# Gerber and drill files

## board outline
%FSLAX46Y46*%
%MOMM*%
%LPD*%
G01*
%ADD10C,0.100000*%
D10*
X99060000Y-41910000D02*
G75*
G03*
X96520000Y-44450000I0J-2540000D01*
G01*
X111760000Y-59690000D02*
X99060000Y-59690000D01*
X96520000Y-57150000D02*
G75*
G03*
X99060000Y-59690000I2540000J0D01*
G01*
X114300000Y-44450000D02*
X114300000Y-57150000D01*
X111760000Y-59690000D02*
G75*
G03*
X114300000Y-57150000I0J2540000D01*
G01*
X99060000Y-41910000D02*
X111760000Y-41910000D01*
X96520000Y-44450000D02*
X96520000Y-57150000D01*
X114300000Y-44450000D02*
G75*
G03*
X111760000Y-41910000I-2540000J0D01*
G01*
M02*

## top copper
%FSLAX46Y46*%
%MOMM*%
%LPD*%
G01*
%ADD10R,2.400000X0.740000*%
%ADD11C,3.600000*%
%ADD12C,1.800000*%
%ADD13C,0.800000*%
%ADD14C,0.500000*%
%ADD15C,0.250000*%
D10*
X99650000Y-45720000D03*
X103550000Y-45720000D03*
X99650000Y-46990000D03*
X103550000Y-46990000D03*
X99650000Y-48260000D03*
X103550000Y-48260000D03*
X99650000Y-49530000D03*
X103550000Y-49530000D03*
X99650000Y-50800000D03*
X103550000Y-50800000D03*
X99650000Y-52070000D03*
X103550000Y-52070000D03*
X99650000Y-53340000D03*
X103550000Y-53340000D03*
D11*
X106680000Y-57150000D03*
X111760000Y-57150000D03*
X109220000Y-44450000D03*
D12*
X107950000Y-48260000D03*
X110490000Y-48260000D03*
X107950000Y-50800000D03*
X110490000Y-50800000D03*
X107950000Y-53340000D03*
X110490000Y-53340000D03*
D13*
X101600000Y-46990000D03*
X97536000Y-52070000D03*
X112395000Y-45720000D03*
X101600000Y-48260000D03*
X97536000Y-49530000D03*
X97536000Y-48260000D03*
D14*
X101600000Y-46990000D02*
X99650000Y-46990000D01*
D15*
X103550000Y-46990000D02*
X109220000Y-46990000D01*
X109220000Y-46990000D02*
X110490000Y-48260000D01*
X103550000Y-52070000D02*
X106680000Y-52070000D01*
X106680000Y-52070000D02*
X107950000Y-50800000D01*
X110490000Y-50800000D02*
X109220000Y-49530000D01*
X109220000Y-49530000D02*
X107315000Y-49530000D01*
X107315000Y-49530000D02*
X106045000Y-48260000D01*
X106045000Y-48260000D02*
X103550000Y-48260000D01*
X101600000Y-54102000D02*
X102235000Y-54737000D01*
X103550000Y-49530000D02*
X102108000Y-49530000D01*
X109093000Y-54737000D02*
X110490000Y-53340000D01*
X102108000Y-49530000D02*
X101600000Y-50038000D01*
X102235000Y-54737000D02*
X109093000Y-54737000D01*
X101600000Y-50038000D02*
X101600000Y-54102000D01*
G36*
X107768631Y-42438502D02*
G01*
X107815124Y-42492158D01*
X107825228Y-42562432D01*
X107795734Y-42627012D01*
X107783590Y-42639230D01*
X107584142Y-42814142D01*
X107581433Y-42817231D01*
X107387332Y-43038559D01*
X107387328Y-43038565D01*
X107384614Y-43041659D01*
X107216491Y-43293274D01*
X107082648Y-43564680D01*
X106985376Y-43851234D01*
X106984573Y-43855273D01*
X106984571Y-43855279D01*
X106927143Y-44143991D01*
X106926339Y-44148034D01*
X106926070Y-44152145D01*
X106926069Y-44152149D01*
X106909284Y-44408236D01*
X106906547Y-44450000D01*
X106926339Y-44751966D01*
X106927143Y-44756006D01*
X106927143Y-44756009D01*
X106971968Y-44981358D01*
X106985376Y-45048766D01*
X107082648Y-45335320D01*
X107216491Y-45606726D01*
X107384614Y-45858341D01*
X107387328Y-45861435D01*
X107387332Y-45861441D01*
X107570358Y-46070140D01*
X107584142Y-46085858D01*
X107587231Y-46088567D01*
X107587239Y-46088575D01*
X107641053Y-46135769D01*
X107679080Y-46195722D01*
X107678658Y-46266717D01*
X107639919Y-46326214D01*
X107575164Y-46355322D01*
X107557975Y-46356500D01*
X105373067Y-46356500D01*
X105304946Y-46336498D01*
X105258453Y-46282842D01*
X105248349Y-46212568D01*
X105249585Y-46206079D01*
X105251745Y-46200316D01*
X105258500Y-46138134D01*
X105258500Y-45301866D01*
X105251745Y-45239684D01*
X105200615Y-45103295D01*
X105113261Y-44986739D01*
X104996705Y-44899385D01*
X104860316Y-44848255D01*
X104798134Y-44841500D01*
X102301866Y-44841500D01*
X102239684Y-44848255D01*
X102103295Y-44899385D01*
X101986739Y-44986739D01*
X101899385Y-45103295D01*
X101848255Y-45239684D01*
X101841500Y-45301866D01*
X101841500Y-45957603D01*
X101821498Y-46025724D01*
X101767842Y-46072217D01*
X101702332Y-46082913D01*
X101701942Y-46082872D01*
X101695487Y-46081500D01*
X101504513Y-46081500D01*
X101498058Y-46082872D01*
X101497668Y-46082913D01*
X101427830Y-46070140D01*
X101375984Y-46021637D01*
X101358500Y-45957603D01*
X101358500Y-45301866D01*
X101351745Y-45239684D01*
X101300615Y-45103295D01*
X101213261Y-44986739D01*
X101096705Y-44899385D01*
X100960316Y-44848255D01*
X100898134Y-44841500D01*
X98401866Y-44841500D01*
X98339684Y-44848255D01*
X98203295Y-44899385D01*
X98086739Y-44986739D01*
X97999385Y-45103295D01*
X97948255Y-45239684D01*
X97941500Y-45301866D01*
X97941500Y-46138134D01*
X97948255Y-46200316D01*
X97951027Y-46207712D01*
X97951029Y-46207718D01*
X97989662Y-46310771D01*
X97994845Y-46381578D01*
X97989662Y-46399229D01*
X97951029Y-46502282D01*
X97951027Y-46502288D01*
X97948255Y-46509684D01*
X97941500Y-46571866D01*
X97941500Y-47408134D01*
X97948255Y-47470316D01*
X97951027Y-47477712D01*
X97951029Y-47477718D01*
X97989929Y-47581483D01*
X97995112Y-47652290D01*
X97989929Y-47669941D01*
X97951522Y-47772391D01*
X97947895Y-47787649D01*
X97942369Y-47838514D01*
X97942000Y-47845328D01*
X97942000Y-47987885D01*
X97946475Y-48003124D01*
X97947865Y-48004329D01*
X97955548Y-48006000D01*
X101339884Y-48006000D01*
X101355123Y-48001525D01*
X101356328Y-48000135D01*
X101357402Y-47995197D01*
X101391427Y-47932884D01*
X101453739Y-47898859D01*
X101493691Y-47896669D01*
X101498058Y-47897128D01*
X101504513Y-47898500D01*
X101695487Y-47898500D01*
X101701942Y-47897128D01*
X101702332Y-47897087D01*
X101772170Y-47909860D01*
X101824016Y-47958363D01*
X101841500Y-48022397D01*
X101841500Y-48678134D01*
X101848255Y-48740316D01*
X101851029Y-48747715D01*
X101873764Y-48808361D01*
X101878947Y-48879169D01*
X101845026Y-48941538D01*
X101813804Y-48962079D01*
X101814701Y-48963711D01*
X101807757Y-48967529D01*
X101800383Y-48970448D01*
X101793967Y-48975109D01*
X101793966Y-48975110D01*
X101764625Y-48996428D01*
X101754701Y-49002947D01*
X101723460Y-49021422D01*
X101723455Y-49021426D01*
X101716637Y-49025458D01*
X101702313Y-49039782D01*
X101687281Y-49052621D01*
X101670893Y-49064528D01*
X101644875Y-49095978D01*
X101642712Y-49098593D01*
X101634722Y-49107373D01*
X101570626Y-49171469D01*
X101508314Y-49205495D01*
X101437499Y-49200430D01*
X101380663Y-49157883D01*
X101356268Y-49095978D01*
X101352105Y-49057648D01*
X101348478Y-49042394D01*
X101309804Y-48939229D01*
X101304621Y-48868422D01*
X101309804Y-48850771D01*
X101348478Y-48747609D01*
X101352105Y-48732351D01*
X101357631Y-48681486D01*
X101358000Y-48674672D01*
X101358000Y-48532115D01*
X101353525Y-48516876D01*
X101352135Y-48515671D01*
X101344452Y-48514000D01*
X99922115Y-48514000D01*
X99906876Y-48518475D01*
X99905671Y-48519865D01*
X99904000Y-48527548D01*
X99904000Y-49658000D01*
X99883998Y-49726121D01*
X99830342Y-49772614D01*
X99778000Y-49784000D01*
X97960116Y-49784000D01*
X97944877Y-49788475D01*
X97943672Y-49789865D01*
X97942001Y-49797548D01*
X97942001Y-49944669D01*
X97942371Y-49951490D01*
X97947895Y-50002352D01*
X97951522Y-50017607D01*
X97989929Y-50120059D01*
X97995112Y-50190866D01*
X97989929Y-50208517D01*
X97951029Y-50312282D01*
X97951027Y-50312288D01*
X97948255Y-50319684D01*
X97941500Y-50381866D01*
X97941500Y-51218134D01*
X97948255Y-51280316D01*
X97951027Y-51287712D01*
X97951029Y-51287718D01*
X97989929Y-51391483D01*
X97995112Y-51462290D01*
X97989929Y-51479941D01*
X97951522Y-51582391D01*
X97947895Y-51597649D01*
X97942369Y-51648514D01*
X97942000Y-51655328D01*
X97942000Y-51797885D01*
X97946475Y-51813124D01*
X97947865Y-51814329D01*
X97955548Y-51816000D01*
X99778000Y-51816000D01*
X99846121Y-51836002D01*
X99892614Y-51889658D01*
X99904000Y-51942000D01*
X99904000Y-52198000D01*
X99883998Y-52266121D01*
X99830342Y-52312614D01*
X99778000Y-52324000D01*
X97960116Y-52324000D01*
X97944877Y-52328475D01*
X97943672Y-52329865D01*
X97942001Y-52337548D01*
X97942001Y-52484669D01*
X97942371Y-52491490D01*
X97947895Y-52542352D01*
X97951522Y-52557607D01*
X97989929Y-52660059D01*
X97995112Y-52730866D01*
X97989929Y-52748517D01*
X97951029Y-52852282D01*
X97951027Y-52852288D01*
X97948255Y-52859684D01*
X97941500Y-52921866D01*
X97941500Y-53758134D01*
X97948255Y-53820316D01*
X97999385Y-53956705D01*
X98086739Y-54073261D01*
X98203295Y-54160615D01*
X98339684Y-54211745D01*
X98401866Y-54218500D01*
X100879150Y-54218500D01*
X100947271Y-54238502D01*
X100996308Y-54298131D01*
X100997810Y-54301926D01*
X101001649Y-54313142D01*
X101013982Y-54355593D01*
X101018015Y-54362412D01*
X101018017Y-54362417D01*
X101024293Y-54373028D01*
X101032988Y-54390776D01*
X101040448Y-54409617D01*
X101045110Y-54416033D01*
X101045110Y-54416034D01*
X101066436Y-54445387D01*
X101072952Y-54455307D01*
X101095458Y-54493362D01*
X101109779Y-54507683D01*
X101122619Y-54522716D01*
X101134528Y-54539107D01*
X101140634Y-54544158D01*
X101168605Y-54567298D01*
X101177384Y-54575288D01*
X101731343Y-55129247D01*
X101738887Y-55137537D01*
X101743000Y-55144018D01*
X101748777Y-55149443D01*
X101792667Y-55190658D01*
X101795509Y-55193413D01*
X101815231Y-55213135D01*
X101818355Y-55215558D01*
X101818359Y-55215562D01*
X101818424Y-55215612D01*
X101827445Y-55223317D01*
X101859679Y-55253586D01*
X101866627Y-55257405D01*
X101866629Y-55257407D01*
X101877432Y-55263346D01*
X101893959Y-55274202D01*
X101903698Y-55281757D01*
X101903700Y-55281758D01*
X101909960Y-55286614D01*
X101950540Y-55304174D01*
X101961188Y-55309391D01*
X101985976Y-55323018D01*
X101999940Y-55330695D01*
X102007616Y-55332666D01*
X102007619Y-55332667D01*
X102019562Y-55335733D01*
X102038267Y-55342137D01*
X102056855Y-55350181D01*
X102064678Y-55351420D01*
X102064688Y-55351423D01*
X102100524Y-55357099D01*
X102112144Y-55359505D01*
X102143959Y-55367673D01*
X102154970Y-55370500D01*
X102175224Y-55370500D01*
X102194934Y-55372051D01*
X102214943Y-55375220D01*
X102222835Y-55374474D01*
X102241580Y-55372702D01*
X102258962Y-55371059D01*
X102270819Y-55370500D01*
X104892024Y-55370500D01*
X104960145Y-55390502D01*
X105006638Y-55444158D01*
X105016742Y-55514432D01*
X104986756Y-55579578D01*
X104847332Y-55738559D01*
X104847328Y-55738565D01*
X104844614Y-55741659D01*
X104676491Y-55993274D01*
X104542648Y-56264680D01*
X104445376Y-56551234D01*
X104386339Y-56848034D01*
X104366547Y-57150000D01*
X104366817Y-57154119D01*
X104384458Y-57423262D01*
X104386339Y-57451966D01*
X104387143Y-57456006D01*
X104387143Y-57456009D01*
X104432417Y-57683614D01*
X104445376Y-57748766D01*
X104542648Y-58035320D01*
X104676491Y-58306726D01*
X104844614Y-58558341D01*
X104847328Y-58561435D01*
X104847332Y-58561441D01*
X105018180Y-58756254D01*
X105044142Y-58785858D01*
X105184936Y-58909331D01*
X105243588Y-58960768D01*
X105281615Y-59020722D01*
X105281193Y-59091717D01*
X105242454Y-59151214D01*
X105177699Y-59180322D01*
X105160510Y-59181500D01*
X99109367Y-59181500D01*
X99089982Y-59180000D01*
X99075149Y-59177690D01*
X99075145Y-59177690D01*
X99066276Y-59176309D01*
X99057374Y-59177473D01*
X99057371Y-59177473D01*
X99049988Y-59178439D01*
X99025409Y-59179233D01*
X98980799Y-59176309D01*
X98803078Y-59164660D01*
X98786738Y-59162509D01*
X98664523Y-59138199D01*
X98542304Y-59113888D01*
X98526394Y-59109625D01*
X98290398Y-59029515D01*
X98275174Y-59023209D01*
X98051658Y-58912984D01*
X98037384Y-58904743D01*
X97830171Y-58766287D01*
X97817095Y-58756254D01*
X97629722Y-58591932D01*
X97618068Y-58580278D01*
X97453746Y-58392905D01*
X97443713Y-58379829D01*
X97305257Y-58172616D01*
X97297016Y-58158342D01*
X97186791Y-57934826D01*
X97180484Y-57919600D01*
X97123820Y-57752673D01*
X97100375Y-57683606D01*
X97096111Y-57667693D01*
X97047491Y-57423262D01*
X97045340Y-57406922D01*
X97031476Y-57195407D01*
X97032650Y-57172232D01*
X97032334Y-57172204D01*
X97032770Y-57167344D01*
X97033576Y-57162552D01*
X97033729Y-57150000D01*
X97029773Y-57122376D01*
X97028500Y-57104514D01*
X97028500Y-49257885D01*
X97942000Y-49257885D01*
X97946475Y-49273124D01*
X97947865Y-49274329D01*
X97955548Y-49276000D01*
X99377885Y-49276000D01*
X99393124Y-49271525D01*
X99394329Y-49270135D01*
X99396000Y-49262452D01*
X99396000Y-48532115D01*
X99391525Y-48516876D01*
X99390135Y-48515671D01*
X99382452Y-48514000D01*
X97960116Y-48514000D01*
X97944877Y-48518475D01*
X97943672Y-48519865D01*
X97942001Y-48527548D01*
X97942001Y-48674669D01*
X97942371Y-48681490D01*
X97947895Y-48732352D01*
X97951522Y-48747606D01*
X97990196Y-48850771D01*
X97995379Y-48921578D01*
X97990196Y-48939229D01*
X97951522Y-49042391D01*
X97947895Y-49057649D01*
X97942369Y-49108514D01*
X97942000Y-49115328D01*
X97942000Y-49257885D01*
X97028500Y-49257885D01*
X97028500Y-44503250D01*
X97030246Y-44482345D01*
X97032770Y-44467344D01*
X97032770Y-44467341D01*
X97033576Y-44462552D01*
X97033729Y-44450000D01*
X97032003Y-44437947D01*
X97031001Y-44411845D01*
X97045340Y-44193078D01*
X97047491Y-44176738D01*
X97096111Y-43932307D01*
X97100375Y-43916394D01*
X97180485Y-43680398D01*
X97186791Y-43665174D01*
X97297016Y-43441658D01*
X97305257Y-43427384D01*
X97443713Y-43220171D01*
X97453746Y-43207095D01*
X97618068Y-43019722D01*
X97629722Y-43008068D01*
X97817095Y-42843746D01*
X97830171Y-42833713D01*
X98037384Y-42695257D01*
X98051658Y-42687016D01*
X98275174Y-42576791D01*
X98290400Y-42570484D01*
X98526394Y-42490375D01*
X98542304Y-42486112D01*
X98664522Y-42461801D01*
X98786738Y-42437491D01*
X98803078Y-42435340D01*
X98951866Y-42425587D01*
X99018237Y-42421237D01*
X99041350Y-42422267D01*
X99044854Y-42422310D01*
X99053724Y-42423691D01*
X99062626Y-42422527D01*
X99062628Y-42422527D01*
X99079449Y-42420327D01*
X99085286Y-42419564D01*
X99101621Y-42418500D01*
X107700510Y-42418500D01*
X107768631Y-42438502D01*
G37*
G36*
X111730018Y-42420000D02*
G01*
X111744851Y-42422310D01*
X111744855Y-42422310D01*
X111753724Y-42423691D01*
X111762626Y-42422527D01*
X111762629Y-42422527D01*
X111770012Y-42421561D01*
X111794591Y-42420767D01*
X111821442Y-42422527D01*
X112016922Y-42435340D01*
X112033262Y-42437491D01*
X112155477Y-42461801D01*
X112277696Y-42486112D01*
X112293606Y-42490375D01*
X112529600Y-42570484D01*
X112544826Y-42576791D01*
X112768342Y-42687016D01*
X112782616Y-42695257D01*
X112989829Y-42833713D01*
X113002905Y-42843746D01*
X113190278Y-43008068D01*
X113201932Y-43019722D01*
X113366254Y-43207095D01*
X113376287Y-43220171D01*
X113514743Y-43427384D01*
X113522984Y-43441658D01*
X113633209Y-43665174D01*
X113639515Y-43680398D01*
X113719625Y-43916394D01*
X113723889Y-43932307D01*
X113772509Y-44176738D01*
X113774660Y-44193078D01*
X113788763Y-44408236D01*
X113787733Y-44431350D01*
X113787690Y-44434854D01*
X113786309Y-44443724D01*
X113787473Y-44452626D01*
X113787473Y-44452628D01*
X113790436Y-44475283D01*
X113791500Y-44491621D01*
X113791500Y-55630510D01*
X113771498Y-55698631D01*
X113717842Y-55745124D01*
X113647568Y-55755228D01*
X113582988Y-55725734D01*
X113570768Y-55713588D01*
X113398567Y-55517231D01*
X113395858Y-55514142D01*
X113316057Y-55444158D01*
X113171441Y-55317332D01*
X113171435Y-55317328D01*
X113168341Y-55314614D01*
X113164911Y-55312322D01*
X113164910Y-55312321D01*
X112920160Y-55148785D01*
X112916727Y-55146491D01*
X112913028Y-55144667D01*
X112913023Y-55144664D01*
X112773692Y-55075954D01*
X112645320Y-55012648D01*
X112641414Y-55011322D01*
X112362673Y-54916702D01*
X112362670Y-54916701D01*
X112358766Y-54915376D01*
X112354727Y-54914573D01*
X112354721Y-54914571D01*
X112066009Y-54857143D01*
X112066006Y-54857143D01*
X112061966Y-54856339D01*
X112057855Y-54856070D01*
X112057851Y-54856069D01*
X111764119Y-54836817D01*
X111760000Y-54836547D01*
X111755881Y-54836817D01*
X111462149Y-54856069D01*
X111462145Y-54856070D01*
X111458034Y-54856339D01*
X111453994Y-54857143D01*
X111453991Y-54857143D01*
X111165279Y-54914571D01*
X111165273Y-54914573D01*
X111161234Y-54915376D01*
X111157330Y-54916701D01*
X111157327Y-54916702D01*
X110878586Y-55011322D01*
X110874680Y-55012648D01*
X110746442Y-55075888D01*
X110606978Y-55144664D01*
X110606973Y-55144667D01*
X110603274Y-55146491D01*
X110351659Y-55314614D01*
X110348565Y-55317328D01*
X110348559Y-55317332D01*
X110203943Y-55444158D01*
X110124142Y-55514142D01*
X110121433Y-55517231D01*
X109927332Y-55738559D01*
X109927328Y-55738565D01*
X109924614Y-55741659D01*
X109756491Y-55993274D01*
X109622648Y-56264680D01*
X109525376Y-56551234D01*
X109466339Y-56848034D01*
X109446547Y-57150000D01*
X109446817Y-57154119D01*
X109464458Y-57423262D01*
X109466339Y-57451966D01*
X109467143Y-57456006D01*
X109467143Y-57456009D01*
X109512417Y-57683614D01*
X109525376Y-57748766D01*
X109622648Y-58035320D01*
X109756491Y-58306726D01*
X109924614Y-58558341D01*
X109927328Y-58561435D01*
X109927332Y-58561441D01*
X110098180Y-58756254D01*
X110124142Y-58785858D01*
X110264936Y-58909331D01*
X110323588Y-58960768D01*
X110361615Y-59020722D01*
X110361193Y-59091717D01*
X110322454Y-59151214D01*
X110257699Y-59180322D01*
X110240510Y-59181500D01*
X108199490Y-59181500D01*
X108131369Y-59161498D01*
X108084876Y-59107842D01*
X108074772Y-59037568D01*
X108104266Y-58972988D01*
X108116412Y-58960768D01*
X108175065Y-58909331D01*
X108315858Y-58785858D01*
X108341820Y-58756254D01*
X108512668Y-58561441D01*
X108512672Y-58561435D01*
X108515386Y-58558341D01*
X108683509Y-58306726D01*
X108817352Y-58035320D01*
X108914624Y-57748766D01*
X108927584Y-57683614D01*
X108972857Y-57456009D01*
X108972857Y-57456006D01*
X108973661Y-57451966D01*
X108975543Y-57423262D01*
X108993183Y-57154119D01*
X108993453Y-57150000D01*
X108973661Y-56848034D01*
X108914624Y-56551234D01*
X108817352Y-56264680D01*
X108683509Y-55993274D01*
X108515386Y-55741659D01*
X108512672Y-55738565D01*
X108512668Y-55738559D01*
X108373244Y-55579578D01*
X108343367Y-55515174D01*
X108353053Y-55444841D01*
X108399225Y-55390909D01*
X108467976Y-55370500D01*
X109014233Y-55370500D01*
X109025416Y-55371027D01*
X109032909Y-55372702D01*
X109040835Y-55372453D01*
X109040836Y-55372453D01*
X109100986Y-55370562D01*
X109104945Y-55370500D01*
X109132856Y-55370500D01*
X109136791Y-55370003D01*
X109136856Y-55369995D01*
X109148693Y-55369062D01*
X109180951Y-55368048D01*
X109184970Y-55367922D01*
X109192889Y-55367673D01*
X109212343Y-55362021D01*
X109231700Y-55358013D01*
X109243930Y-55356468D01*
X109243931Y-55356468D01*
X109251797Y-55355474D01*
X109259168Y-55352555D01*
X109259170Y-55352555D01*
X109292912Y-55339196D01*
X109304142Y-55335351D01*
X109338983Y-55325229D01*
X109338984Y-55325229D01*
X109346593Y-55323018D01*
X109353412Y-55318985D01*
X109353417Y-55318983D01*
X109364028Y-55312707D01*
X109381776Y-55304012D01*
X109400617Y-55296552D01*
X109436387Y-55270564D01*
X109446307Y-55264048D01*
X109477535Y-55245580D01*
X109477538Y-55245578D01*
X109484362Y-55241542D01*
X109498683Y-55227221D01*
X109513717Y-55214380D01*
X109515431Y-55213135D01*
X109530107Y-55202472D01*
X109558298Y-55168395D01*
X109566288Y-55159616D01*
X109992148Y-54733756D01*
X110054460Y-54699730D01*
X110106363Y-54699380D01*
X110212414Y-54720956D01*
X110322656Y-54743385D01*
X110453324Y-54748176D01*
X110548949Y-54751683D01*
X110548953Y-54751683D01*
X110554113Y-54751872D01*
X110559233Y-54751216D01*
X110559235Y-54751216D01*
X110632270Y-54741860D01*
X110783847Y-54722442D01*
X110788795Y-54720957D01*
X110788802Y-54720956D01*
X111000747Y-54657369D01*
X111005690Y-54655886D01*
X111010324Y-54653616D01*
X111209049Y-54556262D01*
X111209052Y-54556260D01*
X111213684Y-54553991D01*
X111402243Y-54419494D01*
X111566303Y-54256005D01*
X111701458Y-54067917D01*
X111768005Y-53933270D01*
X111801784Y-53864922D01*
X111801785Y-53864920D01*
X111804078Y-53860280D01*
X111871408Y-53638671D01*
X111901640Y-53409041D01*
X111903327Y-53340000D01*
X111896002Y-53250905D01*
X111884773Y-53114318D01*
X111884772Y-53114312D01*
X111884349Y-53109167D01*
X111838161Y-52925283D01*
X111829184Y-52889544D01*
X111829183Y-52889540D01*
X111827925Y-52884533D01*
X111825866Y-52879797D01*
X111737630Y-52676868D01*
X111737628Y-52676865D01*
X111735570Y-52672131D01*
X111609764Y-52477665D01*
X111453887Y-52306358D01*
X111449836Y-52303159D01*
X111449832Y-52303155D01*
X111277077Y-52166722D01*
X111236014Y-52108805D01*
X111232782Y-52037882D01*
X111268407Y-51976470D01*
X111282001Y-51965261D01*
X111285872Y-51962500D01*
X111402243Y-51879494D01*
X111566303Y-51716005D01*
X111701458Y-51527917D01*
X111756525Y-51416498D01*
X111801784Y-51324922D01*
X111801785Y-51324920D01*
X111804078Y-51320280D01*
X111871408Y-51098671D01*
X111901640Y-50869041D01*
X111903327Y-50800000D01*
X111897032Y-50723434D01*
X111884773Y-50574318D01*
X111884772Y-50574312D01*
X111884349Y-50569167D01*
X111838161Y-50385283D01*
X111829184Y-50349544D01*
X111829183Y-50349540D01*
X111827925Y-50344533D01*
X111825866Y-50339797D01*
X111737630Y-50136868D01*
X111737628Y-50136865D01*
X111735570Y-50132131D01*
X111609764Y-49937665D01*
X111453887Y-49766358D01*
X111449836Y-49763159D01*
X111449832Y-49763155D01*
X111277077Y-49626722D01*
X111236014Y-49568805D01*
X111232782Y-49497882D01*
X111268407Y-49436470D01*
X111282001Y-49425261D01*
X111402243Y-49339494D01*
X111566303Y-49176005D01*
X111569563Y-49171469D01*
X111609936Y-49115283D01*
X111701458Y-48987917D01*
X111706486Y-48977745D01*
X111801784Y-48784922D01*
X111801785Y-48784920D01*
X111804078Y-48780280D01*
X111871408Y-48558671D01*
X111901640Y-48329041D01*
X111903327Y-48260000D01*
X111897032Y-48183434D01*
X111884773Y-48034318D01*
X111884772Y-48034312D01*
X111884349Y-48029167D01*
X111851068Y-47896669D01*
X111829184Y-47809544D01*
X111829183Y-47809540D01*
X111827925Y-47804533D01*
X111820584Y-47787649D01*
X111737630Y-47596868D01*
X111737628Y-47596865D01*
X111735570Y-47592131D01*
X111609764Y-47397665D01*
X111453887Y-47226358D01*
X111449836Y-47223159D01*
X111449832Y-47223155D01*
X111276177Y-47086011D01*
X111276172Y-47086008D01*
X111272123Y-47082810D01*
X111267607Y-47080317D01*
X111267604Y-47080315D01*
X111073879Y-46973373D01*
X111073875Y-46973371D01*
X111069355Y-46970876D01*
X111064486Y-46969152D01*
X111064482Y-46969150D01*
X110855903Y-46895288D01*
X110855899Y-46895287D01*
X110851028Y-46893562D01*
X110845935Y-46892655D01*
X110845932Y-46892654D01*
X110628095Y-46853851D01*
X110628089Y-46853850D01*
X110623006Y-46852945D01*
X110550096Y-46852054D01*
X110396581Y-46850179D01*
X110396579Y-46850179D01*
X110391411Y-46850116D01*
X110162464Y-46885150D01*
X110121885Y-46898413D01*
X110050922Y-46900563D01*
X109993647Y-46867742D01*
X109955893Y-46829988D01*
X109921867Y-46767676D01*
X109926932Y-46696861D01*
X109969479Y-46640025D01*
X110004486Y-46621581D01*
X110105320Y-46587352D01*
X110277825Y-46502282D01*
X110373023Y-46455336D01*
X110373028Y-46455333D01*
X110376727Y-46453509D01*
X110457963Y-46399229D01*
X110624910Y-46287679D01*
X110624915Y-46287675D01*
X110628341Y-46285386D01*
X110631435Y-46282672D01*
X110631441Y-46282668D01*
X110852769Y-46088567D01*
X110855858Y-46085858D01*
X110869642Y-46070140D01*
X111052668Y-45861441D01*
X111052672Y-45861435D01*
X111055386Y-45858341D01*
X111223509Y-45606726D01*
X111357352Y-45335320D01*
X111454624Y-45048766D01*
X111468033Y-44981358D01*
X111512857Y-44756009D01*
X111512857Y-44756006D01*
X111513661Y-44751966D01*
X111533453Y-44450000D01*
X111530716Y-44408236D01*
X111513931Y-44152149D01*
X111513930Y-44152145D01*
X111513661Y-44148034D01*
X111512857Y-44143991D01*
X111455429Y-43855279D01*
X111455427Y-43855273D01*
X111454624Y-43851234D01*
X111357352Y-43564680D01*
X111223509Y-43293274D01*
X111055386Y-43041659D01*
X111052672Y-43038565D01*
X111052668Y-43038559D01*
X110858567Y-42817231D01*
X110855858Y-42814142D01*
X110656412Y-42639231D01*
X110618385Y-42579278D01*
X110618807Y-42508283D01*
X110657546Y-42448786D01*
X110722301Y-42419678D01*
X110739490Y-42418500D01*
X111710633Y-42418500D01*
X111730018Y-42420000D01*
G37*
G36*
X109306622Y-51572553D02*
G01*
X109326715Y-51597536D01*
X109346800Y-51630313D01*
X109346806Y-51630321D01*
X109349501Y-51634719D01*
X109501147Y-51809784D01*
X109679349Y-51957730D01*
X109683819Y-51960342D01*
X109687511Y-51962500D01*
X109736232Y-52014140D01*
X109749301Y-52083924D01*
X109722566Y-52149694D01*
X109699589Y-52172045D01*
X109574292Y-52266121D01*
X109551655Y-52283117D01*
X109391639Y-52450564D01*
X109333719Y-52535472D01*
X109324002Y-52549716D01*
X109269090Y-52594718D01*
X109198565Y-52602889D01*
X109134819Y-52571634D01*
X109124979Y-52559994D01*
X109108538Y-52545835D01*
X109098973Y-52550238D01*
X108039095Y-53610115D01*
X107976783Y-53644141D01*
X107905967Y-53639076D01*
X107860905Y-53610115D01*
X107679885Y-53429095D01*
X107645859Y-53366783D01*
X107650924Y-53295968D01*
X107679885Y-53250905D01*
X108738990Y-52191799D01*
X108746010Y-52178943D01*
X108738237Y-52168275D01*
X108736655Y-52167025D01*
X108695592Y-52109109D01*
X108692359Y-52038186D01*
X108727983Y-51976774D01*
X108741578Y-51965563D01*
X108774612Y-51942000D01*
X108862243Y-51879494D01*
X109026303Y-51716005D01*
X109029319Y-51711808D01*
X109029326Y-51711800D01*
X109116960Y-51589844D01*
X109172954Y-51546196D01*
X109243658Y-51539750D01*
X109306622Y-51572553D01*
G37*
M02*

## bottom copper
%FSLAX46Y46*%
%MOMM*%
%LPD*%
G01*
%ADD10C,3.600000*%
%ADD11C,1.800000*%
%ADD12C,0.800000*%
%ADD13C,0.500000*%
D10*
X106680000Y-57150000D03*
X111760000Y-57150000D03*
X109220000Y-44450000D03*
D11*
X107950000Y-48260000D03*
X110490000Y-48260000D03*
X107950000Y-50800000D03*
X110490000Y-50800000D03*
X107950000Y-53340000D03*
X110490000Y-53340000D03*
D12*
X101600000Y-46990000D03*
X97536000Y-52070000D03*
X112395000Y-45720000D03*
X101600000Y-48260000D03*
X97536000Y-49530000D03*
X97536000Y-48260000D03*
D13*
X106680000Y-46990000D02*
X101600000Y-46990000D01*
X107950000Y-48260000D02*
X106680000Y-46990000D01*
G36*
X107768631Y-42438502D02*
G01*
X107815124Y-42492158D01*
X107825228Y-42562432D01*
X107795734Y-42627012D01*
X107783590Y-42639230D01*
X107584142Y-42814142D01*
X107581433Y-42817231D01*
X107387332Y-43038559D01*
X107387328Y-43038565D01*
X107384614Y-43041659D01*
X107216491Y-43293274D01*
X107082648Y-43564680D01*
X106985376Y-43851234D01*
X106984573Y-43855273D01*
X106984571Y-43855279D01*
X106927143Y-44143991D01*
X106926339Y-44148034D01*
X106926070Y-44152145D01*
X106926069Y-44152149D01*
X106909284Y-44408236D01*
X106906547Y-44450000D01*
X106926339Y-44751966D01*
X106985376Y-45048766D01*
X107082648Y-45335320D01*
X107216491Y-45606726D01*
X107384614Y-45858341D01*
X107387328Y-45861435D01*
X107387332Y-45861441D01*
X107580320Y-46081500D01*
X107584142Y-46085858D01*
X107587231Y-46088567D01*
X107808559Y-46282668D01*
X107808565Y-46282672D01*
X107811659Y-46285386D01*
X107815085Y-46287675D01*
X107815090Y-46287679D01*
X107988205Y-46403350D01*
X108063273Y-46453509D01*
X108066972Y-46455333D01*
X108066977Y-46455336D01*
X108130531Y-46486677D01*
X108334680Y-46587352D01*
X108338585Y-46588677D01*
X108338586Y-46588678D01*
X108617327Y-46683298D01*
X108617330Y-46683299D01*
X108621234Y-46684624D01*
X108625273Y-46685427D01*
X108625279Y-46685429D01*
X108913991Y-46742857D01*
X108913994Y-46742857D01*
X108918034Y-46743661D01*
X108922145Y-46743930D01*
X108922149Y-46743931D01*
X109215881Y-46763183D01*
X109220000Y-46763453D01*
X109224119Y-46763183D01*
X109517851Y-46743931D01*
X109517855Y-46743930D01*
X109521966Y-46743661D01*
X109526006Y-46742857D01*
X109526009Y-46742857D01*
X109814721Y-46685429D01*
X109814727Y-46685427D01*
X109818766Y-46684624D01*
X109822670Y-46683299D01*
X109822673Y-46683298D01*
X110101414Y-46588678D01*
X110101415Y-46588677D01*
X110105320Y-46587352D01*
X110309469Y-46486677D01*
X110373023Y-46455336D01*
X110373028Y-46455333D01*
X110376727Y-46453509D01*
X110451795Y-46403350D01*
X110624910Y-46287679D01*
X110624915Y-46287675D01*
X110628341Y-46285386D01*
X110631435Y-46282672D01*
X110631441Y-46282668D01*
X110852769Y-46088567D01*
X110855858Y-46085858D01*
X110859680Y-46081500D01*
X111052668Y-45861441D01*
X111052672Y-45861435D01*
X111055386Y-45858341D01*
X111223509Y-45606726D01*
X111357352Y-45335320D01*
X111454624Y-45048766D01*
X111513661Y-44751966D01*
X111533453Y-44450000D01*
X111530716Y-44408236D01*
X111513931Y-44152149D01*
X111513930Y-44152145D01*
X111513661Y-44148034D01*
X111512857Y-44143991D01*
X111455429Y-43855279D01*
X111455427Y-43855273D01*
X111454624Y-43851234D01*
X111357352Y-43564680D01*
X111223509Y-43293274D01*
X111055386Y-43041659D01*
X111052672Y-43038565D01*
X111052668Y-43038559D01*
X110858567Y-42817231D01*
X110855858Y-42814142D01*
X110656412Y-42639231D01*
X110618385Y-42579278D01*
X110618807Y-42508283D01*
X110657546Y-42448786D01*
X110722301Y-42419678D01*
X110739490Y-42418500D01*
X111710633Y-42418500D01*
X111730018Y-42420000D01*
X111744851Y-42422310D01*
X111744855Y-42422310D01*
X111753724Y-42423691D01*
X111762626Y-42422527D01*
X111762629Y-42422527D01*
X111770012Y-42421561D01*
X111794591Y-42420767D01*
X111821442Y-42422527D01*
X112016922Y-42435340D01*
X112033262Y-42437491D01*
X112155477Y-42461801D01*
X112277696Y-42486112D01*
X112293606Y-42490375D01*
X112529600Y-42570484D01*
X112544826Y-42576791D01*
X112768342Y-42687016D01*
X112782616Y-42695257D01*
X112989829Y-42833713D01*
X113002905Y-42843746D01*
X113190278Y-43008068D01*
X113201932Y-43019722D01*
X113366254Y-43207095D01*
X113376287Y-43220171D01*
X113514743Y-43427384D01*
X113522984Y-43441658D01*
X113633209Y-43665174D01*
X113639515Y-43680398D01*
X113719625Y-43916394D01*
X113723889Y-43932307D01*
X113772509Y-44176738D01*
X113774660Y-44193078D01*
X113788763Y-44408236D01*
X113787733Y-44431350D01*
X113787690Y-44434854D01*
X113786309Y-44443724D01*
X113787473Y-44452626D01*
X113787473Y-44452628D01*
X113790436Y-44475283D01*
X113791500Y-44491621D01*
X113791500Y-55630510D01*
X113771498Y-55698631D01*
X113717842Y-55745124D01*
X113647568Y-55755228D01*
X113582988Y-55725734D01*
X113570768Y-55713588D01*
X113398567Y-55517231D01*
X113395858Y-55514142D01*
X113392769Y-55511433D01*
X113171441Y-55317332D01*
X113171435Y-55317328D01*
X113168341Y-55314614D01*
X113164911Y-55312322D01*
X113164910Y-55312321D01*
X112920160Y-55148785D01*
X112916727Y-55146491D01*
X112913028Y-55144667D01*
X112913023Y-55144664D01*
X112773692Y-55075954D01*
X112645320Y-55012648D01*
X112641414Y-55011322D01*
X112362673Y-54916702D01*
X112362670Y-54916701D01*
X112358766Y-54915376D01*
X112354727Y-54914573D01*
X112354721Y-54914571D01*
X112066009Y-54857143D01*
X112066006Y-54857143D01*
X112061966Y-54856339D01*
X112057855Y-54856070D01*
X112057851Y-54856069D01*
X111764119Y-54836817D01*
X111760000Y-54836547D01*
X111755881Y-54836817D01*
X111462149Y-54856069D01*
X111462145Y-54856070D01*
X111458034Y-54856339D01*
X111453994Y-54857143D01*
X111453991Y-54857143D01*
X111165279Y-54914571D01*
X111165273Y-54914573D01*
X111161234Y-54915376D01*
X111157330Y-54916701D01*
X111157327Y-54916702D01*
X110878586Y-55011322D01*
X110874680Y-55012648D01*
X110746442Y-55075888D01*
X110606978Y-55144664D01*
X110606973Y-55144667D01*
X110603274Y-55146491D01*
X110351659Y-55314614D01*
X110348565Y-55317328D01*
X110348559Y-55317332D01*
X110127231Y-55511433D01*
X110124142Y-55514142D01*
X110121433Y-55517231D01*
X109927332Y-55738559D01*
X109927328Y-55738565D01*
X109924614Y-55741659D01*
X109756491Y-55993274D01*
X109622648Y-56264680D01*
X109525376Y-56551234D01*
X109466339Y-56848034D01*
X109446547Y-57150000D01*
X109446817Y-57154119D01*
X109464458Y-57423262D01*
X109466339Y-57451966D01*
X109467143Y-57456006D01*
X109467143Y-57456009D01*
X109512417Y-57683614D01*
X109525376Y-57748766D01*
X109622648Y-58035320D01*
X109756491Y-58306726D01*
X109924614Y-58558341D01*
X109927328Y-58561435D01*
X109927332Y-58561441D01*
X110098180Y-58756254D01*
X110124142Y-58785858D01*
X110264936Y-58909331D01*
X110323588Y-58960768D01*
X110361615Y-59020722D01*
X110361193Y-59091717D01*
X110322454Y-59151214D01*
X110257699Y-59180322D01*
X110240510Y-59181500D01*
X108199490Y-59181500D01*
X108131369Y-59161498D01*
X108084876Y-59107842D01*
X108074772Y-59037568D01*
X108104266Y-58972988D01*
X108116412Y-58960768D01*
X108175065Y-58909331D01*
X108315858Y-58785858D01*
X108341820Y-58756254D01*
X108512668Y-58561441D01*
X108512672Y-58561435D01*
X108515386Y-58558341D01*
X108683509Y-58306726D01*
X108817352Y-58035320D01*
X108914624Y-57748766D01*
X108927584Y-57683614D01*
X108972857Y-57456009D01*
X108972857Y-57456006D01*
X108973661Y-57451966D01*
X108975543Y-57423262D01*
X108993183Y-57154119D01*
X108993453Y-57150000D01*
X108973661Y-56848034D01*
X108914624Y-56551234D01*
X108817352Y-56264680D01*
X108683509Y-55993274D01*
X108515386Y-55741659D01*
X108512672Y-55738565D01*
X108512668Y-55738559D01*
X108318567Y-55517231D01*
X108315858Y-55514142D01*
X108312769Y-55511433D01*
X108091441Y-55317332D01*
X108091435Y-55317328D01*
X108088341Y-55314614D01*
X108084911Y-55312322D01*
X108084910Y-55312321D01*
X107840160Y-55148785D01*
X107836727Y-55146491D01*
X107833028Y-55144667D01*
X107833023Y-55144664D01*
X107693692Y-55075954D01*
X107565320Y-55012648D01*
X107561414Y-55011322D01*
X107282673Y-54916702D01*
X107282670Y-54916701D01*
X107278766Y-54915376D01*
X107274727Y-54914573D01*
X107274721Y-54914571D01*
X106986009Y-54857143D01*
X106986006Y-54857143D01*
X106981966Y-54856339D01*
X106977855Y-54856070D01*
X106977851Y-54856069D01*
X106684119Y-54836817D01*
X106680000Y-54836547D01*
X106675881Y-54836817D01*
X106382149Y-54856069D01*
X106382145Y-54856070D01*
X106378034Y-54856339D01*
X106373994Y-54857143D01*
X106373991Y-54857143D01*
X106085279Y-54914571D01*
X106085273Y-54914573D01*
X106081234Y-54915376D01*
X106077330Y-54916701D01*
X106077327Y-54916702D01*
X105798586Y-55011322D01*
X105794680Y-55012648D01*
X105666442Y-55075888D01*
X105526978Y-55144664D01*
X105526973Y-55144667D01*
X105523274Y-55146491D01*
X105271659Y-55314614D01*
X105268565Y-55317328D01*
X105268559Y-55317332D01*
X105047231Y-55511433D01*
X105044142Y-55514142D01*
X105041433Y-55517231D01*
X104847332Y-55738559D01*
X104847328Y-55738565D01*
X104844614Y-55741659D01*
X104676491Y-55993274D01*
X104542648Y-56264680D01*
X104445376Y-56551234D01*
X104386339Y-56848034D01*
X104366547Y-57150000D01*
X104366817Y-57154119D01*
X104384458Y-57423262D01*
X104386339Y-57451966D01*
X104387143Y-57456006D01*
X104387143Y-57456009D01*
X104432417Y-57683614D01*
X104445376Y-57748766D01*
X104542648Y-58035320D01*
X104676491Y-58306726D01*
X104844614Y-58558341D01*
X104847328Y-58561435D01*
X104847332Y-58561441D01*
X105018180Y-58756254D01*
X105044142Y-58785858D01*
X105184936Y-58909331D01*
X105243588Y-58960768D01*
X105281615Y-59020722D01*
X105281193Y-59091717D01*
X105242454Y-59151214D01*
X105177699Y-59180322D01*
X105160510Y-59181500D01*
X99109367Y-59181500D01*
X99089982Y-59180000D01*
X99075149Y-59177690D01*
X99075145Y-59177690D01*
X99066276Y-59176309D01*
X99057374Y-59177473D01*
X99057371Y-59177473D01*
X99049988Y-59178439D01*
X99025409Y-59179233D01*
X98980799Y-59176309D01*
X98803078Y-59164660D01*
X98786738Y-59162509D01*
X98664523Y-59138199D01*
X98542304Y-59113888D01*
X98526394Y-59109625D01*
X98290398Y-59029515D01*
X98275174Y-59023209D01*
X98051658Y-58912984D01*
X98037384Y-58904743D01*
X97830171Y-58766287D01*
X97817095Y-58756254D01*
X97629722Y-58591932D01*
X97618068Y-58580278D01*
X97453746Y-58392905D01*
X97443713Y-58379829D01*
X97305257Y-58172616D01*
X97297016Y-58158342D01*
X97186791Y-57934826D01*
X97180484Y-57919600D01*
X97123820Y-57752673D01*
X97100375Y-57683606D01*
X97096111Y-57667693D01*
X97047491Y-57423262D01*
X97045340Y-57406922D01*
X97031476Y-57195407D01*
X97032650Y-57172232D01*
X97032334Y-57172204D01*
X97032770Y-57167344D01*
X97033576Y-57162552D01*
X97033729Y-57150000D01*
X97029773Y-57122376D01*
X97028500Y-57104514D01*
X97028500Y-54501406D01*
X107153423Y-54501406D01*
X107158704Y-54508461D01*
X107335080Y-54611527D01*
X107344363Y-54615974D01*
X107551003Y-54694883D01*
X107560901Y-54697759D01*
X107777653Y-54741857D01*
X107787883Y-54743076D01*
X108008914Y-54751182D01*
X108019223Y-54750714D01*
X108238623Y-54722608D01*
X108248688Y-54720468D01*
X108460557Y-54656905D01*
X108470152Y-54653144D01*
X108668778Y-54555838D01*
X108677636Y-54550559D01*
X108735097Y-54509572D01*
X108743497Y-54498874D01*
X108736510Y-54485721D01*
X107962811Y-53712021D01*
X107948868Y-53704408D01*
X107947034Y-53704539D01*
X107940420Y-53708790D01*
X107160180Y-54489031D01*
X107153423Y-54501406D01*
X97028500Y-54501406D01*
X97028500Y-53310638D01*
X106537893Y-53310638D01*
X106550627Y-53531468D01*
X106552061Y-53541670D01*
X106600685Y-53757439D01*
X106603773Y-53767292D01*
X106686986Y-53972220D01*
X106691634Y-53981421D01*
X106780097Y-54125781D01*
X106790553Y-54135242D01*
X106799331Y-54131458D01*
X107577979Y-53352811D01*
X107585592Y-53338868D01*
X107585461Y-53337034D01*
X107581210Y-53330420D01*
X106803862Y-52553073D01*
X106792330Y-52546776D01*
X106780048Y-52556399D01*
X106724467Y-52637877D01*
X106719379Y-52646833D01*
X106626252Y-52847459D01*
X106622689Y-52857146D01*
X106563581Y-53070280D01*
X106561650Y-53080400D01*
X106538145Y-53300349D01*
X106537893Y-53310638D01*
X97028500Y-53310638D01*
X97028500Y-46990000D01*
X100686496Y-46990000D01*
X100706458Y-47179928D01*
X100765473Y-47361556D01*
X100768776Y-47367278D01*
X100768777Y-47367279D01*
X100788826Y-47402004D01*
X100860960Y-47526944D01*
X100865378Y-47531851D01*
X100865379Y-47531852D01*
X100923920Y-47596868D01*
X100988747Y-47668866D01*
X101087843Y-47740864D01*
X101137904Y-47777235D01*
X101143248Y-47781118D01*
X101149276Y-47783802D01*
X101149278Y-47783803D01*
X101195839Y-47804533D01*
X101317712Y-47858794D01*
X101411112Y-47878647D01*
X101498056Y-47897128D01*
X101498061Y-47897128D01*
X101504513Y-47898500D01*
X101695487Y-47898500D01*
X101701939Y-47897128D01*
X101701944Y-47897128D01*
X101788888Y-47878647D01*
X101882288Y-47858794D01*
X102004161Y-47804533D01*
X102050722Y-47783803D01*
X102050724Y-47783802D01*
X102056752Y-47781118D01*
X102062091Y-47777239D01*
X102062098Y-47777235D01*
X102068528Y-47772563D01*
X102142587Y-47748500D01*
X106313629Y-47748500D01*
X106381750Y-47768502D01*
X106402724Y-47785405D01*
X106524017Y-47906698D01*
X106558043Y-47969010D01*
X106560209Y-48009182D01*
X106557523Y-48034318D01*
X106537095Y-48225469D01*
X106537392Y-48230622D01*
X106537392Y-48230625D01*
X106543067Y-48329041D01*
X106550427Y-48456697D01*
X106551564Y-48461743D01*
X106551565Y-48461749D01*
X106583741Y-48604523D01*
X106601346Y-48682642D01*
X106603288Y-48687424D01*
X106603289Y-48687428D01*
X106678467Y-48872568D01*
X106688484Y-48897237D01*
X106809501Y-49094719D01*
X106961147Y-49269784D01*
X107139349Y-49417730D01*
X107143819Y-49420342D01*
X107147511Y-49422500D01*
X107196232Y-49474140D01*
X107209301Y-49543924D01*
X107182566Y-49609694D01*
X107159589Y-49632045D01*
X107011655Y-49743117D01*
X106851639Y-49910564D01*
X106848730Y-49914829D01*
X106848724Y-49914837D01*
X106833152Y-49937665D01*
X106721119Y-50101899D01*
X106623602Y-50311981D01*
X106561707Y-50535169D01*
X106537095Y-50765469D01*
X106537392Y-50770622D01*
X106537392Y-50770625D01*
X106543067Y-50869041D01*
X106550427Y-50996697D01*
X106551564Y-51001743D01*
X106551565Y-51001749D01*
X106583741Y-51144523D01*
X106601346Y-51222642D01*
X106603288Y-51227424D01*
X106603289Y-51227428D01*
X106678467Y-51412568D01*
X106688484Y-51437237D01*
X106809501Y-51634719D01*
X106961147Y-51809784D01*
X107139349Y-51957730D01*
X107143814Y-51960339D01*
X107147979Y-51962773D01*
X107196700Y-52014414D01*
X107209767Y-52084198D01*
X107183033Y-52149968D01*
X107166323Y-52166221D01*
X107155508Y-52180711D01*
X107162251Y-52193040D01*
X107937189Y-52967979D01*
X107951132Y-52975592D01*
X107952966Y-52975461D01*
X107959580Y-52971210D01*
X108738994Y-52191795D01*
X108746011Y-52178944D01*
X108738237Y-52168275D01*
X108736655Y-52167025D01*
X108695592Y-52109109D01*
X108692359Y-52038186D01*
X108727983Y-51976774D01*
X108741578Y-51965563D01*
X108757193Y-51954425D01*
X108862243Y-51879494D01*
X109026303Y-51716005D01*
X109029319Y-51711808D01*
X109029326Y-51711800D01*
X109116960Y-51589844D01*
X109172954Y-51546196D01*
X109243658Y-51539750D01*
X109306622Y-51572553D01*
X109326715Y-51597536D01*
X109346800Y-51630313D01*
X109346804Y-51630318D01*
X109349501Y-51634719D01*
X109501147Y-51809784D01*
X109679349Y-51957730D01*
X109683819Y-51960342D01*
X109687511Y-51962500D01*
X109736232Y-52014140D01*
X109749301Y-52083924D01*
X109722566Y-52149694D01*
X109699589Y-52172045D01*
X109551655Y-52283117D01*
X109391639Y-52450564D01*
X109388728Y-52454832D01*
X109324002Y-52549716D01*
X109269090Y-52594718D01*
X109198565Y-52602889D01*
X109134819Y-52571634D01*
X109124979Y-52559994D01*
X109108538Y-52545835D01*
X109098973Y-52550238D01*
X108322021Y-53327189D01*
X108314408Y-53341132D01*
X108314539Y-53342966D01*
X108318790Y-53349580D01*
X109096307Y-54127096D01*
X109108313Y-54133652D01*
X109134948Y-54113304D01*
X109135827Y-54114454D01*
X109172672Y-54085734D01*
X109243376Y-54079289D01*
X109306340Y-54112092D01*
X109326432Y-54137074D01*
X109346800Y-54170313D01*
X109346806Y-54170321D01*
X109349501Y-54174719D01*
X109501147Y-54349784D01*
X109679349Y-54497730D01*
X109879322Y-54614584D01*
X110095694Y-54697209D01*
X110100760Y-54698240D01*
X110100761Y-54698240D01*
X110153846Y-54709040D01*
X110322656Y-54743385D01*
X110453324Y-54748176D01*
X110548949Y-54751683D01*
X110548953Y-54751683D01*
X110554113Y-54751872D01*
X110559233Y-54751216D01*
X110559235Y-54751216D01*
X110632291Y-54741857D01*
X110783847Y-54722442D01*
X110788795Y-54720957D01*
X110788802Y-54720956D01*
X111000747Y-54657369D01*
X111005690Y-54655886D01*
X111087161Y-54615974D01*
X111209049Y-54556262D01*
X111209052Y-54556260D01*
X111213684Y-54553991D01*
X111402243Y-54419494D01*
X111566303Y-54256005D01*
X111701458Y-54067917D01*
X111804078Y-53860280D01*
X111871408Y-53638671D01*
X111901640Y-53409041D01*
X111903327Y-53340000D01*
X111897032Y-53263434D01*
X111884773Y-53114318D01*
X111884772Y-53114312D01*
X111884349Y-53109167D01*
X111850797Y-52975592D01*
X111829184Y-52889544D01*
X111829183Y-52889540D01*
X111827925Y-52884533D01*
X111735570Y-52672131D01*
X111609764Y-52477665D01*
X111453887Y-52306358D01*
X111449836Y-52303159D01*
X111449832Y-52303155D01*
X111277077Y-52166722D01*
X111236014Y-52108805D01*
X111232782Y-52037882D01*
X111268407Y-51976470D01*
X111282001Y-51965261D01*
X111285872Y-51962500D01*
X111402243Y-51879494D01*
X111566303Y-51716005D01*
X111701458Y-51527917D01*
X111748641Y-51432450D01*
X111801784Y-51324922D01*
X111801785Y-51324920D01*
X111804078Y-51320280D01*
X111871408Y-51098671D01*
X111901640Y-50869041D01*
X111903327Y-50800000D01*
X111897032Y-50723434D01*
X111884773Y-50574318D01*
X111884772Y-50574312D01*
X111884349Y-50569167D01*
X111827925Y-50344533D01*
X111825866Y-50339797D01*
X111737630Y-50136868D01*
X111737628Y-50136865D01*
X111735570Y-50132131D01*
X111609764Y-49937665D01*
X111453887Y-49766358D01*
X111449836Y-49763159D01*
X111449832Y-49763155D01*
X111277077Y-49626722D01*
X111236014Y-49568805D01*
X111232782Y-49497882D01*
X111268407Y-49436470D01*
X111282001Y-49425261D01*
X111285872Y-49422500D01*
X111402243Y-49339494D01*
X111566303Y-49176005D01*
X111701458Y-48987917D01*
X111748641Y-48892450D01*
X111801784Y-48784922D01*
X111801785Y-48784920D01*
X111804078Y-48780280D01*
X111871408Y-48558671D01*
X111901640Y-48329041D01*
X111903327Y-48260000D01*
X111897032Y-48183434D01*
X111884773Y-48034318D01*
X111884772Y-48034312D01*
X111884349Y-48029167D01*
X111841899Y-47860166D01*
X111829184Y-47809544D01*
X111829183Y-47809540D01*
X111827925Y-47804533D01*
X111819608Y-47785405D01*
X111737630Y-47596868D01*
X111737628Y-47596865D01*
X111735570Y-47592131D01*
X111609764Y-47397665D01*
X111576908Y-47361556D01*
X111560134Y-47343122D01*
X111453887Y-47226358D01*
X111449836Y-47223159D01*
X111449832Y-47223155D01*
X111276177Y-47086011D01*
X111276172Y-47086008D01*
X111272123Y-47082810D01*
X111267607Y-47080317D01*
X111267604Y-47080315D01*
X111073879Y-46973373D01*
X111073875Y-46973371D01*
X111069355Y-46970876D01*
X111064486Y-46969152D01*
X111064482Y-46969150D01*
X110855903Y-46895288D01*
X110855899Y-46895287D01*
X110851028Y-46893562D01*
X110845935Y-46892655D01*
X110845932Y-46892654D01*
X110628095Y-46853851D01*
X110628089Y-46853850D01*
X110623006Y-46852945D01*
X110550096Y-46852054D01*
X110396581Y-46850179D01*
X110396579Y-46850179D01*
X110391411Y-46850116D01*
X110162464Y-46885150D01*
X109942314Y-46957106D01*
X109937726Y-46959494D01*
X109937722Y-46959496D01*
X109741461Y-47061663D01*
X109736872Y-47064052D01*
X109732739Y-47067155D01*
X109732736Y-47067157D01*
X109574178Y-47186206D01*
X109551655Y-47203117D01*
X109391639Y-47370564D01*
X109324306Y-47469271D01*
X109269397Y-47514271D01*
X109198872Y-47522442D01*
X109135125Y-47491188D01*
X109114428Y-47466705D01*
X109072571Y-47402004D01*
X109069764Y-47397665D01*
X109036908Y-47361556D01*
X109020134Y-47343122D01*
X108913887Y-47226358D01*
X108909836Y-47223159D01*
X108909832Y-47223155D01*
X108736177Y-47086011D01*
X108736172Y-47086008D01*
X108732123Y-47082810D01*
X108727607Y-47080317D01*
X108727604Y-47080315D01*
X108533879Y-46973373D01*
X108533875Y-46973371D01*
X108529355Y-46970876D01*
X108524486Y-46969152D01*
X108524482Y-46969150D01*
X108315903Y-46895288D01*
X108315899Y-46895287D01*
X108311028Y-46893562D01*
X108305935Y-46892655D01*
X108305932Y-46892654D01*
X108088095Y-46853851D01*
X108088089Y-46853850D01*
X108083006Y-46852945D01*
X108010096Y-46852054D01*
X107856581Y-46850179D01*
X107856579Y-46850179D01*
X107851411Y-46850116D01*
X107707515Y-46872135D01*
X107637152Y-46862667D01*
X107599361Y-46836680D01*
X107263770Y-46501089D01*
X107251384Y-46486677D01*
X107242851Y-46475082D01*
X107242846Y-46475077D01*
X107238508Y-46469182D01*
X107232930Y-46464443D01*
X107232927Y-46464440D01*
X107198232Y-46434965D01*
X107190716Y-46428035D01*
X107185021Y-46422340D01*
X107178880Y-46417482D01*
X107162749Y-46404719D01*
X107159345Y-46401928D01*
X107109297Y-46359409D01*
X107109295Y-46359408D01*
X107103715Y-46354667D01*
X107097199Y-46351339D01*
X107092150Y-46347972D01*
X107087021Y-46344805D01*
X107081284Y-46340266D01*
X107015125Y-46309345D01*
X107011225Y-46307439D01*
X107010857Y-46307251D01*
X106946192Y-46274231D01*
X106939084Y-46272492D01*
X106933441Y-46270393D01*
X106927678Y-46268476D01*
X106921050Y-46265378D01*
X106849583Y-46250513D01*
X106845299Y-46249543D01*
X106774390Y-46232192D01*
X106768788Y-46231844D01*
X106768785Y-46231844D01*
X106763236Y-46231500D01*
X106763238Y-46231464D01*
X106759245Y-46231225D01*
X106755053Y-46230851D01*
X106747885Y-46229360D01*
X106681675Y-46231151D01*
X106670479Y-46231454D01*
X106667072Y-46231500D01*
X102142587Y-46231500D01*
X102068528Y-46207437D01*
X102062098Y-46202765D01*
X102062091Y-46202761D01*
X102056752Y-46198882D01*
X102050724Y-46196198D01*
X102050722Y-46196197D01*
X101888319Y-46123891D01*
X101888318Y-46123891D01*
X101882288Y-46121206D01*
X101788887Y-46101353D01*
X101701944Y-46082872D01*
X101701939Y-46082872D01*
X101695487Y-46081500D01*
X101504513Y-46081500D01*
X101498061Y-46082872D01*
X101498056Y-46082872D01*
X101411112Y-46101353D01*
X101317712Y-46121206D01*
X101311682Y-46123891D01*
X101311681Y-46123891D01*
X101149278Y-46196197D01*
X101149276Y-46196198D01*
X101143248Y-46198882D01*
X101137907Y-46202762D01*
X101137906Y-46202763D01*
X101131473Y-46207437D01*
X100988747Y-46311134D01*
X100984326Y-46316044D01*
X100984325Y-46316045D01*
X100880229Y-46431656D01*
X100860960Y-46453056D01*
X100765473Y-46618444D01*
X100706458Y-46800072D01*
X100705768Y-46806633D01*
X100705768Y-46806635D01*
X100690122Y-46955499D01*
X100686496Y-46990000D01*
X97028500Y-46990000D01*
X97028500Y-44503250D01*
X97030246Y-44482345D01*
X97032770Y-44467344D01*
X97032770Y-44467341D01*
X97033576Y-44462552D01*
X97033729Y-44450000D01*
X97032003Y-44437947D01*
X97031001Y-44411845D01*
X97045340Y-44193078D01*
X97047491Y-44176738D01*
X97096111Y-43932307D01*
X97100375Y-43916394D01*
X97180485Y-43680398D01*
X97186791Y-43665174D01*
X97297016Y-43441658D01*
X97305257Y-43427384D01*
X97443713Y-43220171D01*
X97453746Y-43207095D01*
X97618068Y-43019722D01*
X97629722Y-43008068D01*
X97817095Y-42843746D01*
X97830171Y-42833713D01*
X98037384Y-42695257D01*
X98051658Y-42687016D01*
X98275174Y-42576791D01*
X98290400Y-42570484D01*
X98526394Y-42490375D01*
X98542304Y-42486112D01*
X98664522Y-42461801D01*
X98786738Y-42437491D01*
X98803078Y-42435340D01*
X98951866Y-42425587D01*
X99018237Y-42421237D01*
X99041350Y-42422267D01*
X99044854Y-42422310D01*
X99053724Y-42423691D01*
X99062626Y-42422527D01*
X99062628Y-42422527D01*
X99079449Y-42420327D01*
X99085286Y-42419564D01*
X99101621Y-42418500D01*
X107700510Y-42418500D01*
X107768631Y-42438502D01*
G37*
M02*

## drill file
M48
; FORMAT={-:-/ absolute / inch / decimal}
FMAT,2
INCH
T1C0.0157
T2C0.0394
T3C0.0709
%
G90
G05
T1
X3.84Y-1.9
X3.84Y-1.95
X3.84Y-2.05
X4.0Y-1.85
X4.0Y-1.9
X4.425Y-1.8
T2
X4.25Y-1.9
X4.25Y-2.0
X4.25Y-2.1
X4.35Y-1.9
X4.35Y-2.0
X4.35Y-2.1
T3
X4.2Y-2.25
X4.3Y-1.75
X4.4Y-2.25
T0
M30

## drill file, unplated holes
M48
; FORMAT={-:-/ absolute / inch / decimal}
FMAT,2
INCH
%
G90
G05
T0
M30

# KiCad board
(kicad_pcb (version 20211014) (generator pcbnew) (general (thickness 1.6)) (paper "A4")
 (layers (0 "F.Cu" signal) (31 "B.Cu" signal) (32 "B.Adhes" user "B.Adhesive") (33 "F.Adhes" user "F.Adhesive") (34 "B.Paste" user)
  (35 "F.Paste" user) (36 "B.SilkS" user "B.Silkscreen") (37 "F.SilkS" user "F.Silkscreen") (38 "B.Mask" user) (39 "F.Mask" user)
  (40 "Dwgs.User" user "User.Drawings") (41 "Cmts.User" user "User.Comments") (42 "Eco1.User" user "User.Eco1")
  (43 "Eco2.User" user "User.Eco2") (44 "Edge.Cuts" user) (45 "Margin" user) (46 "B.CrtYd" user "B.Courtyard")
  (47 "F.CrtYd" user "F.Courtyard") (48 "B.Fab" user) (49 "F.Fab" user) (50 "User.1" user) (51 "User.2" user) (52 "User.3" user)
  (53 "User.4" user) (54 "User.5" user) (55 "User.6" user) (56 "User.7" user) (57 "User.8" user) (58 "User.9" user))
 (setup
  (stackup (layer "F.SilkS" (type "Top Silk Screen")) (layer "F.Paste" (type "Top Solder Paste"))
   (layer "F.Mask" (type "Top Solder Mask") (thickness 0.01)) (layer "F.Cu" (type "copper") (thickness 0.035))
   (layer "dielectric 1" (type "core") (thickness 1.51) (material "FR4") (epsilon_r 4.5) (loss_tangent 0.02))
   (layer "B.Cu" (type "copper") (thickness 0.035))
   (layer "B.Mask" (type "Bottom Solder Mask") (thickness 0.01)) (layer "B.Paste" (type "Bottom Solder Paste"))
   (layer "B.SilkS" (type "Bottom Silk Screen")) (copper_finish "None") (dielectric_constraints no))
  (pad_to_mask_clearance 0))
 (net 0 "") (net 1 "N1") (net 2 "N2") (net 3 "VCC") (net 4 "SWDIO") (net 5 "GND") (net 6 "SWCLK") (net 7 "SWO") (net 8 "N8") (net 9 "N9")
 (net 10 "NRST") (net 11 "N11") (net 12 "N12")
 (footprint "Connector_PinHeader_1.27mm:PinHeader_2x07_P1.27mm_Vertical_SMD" (layer "F.Cu") (at 101.6 49.53)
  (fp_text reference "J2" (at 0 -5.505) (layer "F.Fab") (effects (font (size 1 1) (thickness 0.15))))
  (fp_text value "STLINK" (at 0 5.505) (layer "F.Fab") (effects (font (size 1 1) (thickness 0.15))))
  (pad "1" smd rect (at -1.95 -3.81) (size 2.4 0.74) (layers "F.Cu" "F.Paste" "F.Mask") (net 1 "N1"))
  (pad "2" smd rect (at 1.95 -3.81) (size 2.4 0.74) (layers "F.Cu" "F.Paste" "F.Mask") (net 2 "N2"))
  (pad "3" smd rect (at -1.95 -2.54) (size 2.4 0.74) (layers "F.Cu" "F.Paste" "F.Mask") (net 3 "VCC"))
  (pad "4" smd rect (at 1.95 -2.54) (size 2.4 0.74) (layers "F.Cu" "F.Paste" "F.Mask") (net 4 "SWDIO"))
  (pad "5" smd rect (at -1.95 -1.27) (size 2.4 0.74) (layers "F.Cu" "F.Paste" "F.Mask") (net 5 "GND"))
  (pad "6" smd rect (at 1.95 -1.27) (size 2.4 0.74) (layers "F.Cu" "F.Paste" "F.Mask") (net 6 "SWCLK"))
  (pad "7" smd rect (at -1.95 0) (size 2.4 0.74) (layers "F.Cu" "F.Paste" "F.Mask") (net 5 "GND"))
  (pad "8" smd rect (at 1.95 0) (size 2.4 0.74) (layers "F.Cu" "F.Paste" "F.Mask") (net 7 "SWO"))
  (pad "9" smd rect (at -1.95 1.27) (size 2.4 0.74) (layers "F.Cu" "F.Paste" "F.Mask") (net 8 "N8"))
  (pad "10" smd rect (at 1.95 1.27) (size 2.4 0.74) (layers "F.Cu" "F.Paste" "F.Mask") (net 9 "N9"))
  (pad "11" smd rect (at -1.95 2.54) (size 2.4 0.74) (layers "F.Cu" "F.Paste" "F.Mask") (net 5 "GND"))
  (pad "12" smd rect (at 1.95 2.54) (size 2.4 0.74) (layers "F.Cu" "F.Paste" "F.Mask") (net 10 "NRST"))
  (pad "13" smd rect (at -1.95 3.81) (size 2.4 0.74) (layers "F.Cu" "F.Paste" "F.Mask") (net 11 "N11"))
  (pad "14" smd rect (at 1.95 3.81) (size 2.4 0.74) (layers "F.Cu" "F.Paste" "F.Mask") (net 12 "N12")))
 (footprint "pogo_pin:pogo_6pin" (layer "F.Cu") (at 109.22 50.8)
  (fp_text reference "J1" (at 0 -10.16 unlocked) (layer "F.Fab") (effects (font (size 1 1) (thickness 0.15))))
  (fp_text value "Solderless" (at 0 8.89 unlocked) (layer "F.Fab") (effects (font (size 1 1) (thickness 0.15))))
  (pad "" thru_hole circle (at -2.54 6.35) (size 3.6 3.6) (drill 1.8) (layers *.Cu *.Mask))
  (pad "" thru_hole circle (at 2.54 6.35) (size 3.6 3.6) (drill 1.8) (layers *.Cu *.Mask))
  (pad "" thru_hole circle (at 0 -6.35) (size 3.6 3.6) (drill 1.8) (layers *.Cu *.Mask))
  (pad "1" thru_hole circle (at -1.27 -2.54) (size 1.8 1.8) (drill 1) (layers *.Cu *.Mask) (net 3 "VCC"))
  (pad "2" thru_hole circle (at 1.27 -2.54) (size 1.8 1.8) (drill 1) (layers *.Cu *.Mask) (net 4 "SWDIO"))
  (pad "3" thru_hole circle (at -1.27 0) (size 1.8 1.8) (drill 1) (layers *.Cu *.Mask) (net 10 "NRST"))
  (pad "4" thru_hole circle (at 1.27 0) (size 1.8 1.8) (drill 1) (layers *.Cu *.Mask) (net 6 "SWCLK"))
  (pad "5" thru_hole circle (at -1.27 2.54) (size 1.8 1.8) (drill 1) (layers *.Cu *.Mask) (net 5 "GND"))
  (pad "6" thru_hole circle (at 1.27 2.54) (size 1.8 1.8) (drill 1) (layers *.Cu *.Mask) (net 7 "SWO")))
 (gr_arc (start 96.52 44.45) (mid 97.263949 42.653949) (end 99.06 41.91) (layer "Edge.Cuts") (width 0.1))
 (gr_line (start 111.76 59.69) (end 99.06 59.69) (layer "Edge.Cuts") (width 0.1))
 (gr_arc (start 99.06 59.69) (mid 97.263949 58.946051) (end 96.52 57.15) (layer "Edge.Cuts") (width 0.1))
 (gr_line (start 114.3 44.45) (end 114.3 57.15) (layer "Edge.Cuts") (width 0.1))
 (gr_arc (start 114.3 57.15) (mid 113.556051 58.946051) (end 111.76 59.69) (layer "Edge.Cuts") (width 0.1))
 (gr_line (start 99.06 41.91) (end 111.76 41.91) (layer "Edge.Cuts") (width 0.1))
 (gr_line (start 96.52 44.45) (end 96.52 57.15) (layer "Edge.Cuts") (width 0.1))
 (gr_arc (start 111.76 41.91) (mid 113.556051 42.653949) (end 114.3 44.45) (layer "Edge.Cuts") (width 0.1))
 (segment (start 101.6 46.99) (end 99.65 46.99) (width 0.5) (layer "F.Cu") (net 3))
 (via (at 101.6 46.99) (size 0.8) (drill 0.4) (layers "F.Cu" "B.Cu") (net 3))
 (segment (start 106.68 46.99) (end 101.6 46.99) (width 0.5) (layer "B.Cu") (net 3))
 (segment (start 107.95 48.26) (end 106.68 46.99) (width 0.5) (layer "B.Cu") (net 3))
 (segment (start 103.55 46.99) (end 109.22 46.99) (width 0.25) (layer "F.Cu") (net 4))
 (segment (start 109.22 46.99) (end 110.49 48.26) (width 0.25) (layer "F.Cu") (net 4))
 (segment (start 103.55 52.07) (end 106.68 52.07) (width 0.25) (layer "F.Cu") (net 10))
 (segment (start 106.68 52.07) (end 107.95 50.8) (width 0.25) (layer "F.Cu") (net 10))
 (segment (start 110.49 50.8) (end 109.22 49.53) (width 0.25) (layer "F.Cu") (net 6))
 (segment (start 109.22 49.53) (end 107.315 49.53) (width 0.25) (layer "F.Cu") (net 6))
 (segment (start 107.315 49.53) (end 106.045 48.26) (width 0.25) (layer "F.Cu") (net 6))
 (segment (start 106.045 48.26) (end 103.55 48.26) (width 0.25) (layer "F.Cu") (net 6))
 (via (at 97.536 52.07) (size 0.8) (drill 0.4) (layers "F.Cu" "B.Cu") (free) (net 5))
 (via (at 112.395 45.72) (size 0.8) (drill 0.4) (layers "F.Cu" "B.Cu") (free) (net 5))
 (via (at 101.6 48.26) (size 0.8) (drill 0.4) (layers "F.Cu" "B.Cu") (free) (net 5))
 (via (at 97.536 49.53) (size 0.8) (drill 0.4) (layers "F.Cu" "B.Cu") (free) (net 5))
 (via (at 97.536 48.26) (size 0.8) (drill 0.4) (layers "F.Cu" "B.Cu") (free) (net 5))
 (segment (start 101.6 54.102) (end 102.235 54.737) (width 0.25) (layer "F.Cu") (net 7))
 (segment (start 103.55 49.53) (end 102.108 49.53) (width 0.25) (layer "F.Cu") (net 7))
 (segment (start 109.093 54.737) (end 110.49 53.34) (width 0.25) (layer "F.Cu") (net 7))
 (segment (start 102.108 49.53) (end 101.6 50.038) (width 0.25) (layer "F.Cu") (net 7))
 (segment (start 102.235 54.737) (end 109.093 54.737) (width 0.25) (layer "F.Cu") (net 7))
 (segment (start 101.6 50.038) (end 101.6 54.102) (width 0.25) (layer "F.Cu") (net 7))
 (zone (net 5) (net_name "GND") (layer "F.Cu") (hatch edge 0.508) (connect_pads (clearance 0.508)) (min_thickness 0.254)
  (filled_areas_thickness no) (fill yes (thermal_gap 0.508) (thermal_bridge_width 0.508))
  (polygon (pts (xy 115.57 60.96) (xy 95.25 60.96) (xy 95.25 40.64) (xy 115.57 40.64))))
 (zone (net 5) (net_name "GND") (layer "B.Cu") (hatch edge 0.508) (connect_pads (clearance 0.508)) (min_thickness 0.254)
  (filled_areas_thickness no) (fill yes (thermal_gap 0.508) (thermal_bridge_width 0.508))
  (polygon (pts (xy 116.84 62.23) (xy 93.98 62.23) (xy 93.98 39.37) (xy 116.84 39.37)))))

